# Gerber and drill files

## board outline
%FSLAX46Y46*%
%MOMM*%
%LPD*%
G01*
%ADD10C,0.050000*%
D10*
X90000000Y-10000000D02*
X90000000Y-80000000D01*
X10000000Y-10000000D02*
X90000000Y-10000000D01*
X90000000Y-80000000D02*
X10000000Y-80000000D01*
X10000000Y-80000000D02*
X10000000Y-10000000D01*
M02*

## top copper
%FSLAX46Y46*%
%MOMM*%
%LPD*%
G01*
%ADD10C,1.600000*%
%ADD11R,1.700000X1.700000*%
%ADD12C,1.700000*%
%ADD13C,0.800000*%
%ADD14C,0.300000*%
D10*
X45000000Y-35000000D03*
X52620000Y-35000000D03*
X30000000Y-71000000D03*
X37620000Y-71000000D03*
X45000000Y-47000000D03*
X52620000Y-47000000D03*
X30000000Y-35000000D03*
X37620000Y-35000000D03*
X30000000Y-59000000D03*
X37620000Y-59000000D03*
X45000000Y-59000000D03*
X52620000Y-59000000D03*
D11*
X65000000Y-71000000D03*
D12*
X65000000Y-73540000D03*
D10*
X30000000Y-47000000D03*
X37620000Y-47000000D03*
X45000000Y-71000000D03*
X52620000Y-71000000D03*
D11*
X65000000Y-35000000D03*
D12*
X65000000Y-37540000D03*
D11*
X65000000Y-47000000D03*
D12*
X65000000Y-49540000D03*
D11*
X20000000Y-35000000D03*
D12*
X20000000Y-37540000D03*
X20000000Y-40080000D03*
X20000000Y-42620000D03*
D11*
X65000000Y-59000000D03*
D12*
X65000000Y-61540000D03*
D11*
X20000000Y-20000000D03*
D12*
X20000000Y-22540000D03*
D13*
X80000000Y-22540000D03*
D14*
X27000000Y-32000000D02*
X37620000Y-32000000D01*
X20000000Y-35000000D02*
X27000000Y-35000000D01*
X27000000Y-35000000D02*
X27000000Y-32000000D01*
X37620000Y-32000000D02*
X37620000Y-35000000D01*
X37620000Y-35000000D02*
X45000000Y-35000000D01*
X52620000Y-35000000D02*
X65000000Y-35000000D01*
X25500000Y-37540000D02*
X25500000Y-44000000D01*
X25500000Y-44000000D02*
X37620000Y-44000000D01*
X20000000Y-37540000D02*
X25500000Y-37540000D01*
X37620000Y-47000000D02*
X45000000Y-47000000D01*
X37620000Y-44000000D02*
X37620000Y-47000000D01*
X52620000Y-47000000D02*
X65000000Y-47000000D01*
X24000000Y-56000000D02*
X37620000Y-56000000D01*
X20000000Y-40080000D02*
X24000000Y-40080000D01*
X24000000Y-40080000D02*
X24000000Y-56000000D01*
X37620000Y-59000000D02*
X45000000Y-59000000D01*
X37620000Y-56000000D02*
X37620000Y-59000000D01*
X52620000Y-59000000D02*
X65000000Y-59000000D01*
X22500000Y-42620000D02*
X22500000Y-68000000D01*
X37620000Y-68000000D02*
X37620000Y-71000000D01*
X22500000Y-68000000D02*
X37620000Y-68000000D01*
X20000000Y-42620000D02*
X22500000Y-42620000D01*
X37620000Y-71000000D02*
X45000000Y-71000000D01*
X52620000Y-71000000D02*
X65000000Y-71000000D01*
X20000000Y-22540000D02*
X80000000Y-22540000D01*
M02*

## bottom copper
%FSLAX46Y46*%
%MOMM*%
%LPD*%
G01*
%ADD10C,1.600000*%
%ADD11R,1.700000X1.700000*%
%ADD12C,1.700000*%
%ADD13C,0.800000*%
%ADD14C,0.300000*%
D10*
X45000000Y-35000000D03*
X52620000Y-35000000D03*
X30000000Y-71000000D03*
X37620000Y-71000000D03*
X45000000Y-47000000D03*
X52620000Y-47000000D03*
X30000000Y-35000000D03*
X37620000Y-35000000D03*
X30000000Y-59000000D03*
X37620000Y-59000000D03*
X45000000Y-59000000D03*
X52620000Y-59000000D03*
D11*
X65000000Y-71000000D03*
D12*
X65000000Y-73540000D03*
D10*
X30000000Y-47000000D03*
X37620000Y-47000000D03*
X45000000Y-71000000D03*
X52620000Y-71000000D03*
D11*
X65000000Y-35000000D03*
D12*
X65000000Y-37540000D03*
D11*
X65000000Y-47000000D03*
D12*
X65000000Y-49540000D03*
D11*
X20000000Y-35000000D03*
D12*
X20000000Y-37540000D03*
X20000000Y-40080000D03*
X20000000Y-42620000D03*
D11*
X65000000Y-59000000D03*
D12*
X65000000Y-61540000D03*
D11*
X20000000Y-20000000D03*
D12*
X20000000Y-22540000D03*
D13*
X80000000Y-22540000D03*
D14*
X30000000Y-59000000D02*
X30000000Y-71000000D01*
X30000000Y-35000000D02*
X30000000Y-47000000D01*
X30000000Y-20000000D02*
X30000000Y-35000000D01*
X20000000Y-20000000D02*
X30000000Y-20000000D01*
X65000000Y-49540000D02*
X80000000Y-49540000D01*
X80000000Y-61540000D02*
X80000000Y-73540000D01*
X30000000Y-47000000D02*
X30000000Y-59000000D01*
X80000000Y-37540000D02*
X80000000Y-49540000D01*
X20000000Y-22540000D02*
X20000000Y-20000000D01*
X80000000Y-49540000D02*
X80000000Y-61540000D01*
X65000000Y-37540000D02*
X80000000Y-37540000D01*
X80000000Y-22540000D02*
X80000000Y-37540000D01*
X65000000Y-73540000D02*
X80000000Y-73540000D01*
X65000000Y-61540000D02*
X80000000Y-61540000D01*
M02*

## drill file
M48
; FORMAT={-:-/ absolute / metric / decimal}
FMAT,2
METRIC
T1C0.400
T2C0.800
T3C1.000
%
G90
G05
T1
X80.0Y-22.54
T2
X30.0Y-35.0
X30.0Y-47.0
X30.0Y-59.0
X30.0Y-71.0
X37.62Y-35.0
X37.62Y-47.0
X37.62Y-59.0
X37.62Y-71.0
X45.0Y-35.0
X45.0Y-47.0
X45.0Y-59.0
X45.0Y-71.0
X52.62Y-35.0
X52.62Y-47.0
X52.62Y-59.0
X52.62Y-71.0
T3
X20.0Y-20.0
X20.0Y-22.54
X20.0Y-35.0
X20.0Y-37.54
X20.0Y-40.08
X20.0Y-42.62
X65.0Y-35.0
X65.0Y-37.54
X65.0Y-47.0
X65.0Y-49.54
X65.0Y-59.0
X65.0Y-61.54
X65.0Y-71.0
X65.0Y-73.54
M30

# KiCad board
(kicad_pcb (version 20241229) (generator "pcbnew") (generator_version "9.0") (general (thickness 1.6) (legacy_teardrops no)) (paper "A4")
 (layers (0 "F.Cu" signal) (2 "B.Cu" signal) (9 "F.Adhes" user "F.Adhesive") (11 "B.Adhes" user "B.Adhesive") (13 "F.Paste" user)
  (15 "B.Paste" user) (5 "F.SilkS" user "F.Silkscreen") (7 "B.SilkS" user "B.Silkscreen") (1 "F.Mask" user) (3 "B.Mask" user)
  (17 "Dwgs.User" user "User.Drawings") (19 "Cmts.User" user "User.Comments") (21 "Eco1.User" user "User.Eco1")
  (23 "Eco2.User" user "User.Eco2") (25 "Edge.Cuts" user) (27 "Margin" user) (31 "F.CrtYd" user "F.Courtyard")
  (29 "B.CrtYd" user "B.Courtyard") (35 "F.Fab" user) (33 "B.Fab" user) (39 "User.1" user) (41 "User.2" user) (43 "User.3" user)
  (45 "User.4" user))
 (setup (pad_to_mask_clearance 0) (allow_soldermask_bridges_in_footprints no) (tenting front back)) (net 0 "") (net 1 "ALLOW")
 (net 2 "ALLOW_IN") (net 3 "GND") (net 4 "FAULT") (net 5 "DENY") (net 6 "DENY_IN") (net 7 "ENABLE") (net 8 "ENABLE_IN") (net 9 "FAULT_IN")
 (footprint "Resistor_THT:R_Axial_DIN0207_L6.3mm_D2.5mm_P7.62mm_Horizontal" (layer "F.Cu") (at 45 35)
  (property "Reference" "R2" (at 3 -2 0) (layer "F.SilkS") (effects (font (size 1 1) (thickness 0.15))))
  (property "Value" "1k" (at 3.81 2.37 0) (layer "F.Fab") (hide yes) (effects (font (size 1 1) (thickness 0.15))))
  (pad "1" thru_hole circle (at 0 0) (size 1.6 1.6) (drill 0.8) (layers "*.Cu" "*.Mask") (remove_unused_layers no) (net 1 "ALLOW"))
  (pad "2" thru_hole circle (at 7.62 0) (size 1.6 1.6) (drill 0.8) (layers "*.Cu" "*.Mask") (remove_unused_layers no) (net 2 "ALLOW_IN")))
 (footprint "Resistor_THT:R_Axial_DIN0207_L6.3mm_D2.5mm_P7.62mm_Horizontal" (layer "F.Cu") (at 30 71)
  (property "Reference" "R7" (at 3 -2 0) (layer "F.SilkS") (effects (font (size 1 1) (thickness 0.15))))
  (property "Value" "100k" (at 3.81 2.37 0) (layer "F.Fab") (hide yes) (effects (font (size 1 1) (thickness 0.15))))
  (pad "1" thru_hole circle (at 0 0) (size 1.6 1.6) (drill 0.8) (layers "*.Cu" "*.Mask") (remove_unused_layers no) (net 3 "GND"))
  (pad "2" thru_hole circle (at 7.62 0) (size 1.6 1.6) (drill 0.8) (layers "*.Cu" "*.Mask") (remove_unused_layers no) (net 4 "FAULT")))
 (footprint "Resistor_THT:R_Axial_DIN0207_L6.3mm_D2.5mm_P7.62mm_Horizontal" (layer "F.Cu") (at 45 47)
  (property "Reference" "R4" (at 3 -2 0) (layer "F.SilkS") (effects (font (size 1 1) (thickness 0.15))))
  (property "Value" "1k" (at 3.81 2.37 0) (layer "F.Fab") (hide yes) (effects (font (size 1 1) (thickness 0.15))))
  (pad "1" thru_hole circle (at 0 0) (size 1.6 1.6) (drill 0.8) (layers "*.Cu" "*.Mask") (remove_unused_layers no) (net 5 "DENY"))
  (pad "2" thru_hole circle (at 7.62 0) (size 1.6 1.6) (drill 0.8) (layers "*.Cu" "*.Mask") (remove_unused_layers no) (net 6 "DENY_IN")))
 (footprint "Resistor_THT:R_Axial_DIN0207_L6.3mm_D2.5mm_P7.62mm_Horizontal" (layer "F.Cu") (at 30 35)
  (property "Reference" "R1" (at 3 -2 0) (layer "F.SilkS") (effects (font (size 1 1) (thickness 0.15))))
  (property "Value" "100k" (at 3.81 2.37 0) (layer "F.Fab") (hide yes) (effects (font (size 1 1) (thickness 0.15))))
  (pad "1" thru_hole circle (at 0 0) (size 1.6 1.6) (drill 0.8) (layers "*.Cu" "*.Mask") (remove_unused_layers no) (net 3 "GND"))
  (pad "2" thru_hole circle (at 7.62 0) (size 1.6 1.6) (drill 0.8) (layers "*.Cu" "*.Mask") (remove_unused_layers no) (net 1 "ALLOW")))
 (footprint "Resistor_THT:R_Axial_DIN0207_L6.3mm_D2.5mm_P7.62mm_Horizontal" (layer "F.Cu") (at 30 59)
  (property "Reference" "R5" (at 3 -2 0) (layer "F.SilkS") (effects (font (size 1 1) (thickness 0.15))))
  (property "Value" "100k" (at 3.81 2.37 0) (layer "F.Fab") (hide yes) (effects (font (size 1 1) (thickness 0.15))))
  (pad "1" thru_hole circle (at 0 0) (size 1.6 1.6) (drill 0.8) (layers "*.Cu" "*.Mask") (remove_unused_layers no) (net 3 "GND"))
  (pad "2" thru_hole circle (at 7.62 0) (size 1.6 1.6) (drill 0.8) (layers "*.Cu" "*.Mask") (remove_unused_layers no) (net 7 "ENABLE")))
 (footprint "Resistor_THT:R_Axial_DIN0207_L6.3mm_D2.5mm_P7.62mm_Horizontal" (layer "F.Cu") (at 45 59)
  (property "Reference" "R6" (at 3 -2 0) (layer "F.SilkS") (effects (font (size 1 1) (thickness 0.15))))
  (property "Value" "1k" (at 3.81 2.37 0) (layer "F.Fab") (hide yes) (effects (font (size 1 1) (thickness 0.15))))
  (pad "1" thru_hole circle (at 0 0) (size 1.6 1.6) (drill 0.8) (layers "*.Cu" "*.Mask") (remove_unused_layers no) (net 7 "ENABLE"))
  (pad "2" thru_hole circle (at 7.62 0) (size 1.6 1.6) (drill 0.8) (layers "*.Cu" "*.Mask") (remove_unused_layers no) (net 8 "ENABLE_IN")))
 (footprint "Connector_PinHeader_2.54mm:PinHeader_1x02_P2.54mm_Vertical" (layer "F.Cu") (at 65 71)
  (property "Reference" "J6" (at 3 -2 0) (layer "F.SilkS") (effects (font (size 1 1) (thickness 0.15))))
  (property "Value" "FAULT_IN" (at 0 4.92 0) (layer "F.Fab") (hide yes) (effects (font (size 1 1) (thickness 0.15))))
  (pad "1" thru_hole rect (at 0 0) (size 1.7 1.7) (drill 1) (layers "*.Cu" "*.Mask") (remove_unused_layers no) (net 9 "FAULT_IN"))
  (pad "2" thru_hole circle (at 0 2.54) (size 1.7 1.7) (drill 1) (layers "*.Cu" "*.Mask") (remove_unused_layers no) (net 3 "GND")))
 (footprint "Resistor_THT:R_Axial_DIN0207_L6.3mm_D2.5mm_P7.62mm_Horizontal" (layer "F.Cu") (at 30 47)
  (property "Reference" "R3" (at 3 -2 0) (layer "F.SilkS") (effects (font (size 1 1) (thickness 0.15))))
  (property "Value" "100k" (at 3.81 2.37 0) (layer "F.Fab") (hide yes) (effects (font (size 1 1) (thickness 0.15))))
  (pad "1" thru_hole circle (at 0 0) (size 1.6 1.6) (drill 0.8) (layers "*.Cu" "*.Mask") (remove_unused_layers no) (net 3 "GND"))
  (pad "2" thru_hole circle (at 7.62 0) (size 1.6 1.6) (drill 0.8) (layers "*.Cu" "*.Mask") (remove_unused_layers no) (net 5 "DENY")))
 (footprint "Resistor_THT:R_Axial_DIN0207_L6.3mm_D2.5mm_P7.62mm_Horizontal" (layer "F.Cu") (at 45 71)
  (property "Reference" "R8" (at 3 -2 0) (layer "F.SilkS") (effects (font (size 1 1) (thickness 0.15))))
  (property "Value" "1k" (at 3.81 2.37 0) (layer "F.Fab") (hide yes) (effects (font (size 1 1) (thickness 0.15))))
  (pad "1" thru_hole circle (at 0 0) (size 1.6 1.6) (drill 0.8) (layers "*.Cu" "*.Mask") (remove_unused_layers no) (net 4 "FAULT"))
  (pad "2" thru_hole circle (at 7.62 0) (size 1.6 1.6) (drill 0.8) (layers "*.Cu" "*.Mask") (remove_unused_layers no) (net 9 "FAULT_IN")))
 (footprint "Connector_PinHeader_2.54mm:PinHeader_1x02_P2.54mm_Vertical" (layer "F.Cu") (at 65 35)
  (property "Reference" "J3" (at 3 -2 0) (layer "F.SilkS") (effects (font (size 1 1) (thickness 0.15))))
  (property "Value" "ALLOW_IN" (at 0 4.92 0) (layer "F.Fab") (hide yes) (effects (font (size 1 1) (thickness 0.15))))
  (pad "1" thru_hole rect (at 0 0) (size 1.7 1.7) (drill 1) (layers "*.Cu" "*.Mask") (remove_unused_layers no) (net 2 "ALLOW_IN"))
  (pad "2" thru_hole circle (at 0 2.54) (size 1.7 1.7) (drill 1) (layers "*.Cu" "*.Mask") (remove_unused_layers no) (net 3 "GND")))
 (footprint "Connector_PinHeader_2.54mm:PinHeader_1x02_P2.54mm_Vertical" (layer "F.Cu") (at 65 47)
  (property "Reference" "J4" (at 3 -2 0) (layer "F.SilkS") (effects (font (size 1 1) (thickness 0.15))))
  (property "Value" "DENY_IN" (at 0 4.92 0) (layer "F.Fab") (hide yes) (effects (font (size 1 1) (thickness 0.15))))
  (pad "1" thru_hole rect (at 0 0) (size 1.7 1.7) (drill 1) (layers "*.Cu" "*.Mask") (remove_unused_layers no) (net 6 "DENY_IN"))
  (pad "2" thru_hole circle (at 0 2.54) (size 1.7 1.7) (drill 1) (layers "*.Cu" "*.Mask") (remove_unused_layers no) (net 3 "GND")))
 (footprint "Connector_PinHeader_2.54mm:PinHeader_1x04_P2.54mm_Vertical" (layer "F.Cu") (at 20 35)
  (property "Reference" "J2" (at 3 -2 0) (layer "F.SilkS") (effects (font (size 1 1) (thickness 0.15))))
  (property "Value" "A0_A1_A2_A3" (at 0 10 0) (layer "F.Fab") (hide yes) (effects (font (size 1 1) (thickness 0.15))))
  (pad "1" thru_hole rect (at 0 0) (size 1.7 1.7) (drill 1) (layers "*.Cu" "*.Mask") (remove_unused_layers no) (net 1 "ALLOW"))
  (pad "2" thru_hole circle (at 0 2.54) (size 1.7 1.7) (drill 1) (layers "*.Cu" "*.Mask") (remove_unused_layers no) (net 5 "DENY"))
  (pad "3" thru_hole circle (at 0 5.08) (size 1.7 1.7) (drill 1) (layers "*.Cu" "*.Mask") (remove_unused_layers no) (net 7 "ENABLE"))
  (pad "4" thru_hole circle (at 0 7.62) (size 1.7 1.7) (drill 1) (layers "*.Cu" "*.Mask") (remove_unused_layers no) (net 4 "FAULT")))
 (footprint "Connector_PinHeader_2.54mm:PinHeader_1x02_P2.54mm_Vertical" (layer "F.Cu") (at 65 59)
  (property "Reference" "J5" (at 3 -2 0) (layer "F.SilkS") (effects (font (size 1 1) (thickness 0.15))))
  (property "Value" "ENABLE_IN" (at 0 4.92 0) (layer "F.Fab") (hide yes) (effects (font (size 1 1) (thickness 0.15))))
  (pad "1" thru_hole rect (at 0 0) (size 1.7 1.7) (drill 1) (layers "*.Cu" "*.Mask") (remove_unused_layers no) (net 8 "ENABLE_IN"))
  (pad "2" thru_hole circle (at 0 2.54) (size 1.7 1.7) (drill 1) (layers "*.Cu" "*.Mask") (remove_unused_layers no) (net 3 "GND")))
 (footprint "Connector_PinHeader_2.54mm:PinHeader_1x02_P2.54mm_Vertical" (layer "F.Cu") (at 20 20)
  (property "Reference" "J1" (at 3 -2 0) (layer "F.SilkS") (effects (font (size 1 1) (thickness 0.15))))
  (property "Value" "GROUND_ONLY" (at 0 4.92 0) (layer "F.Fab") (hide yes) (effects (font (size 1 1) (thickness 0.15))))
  (pad "1" thru_hole rect (at 0 0) (size 1.7 1.7) (drill 1) (layers "*.Cu" "*.Mask") (remove_unused_layers no) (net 3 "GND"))
  (pad "2" thru_hole circle (at 0 2.54) (size 1.7 1.7) (drill 1) (layers "*.Cu" "*.Mask") (remove_unused_layers no) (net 3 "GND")))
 (gr_line (start 90 10) (end 90 80) (stroke (width 0.05) (type default)) (layer "Edge.Cuts"))
 (gr_line (start 10 10) (end 90 10) (stroke (width 0.05) (type default)) (layer "Edge.Cuts"))
 (gr_line (start 90 80) (end 10 80) (stroke (width 0.05) (type default)) (layer "Edge.Cuts"))
 (gr_line (start 10 80) (end 10 10) (stroke (width 0.05) (type default)) (layer "Edge.Cuts"))
 (segment (start 27 32) (end 37.62 32) (width 0.3) (layer "F.Cu") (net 1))
 (segment (start 20 35) (end 27 35) (width 0.3) (layer "F.Cu") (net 1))
 (segment (start 27 35) (end 27 32) (width 0.3) (layer "F.Cu") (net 1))
 (segment (start 37.62 32) (end 37.62 35) (width 0.3) (layer "F.Cu") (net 1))
 (segment (start 37.62 35) (end 45 35) (width 0.3) (layer "F.Cu") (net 1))
 (segment (start 52.62 35) (end 65 35) (width 0.3) (layer "F.Cu") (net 2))
 (segment (start 25.5 37.54) (end 25.5 44) (width 0.3) (layer "F.Cu") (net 5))
 (segment (start 25.5 44) (end 37.62 44) (width 0.3) (layer "F.Cu") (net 5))
 (segment (start 20 37.54) (end 25.5 37.54) (width 0.3) (layer "F.Cu") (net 5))
 (segment (start 37.62 47) (end 45 47) (width 0.3) (layer "F.Cu") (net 5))
 (segment (start 37.62 44) (end 37.62 47) (width 0.3) (layer "F.Cu") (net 5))
 (segment (start 52.62 47) (end 65 47) (width 0.3) (layer "F.Cu") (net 6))
 (segment (start 24 56) (end 37.62 56) (width 0.3) (layer "F.Cu") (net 7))
 (segment (start 20 40.08) (end 24 40.08) (width 0.3) (layer "F.Cu") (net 7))
 (segment (start 24 40.08) (end 24 56) (width 0.3) (layer "F.Cu") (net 7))
 (segment (start 37.62 59) (end 45 59) (width 0.3) (layer "F.Cu") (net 7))
 (segment (start 37.62 56) (end 37.62 59) (width 0.3) (layer "F.Cu") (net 7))
 (segment (start 52.62 59) (end 65 59) (width 0.3) (layer "F.Cu") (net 8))
 (segment (start 22.5 42.62) (end 22.5 68) (width 0.3) (layer "F.Cu") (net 4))
 (segment (start 37.62 68) (end 37.62 71) (width 0.3) (layer "F.Cu") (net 4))
 (segment (start 22.5 68) (end 37.62 68) (width 0.3) (layer "F.Cu") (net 4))
 (segment (start 20 42.62) (end 22.5 42.62) (width 0.3) (layer "F.Cu") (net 4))
 (segment (start 37.62 71) (end 45 71) (width 0.3) (layer "F.Cu") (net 4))
 (segment (start 52.62 71) (end 65 71) (width 0.3) (layer "F.Cu") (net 9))
 (segment (start 20 22.54) (end 80 22.54) (width 0.3) (layer "F.Cu") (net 3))
 (via (at 80 22.54) (size 0.8) (drill 0.4) (layers "F.Cu" "B.Cu") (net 3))
 (segment (start 30 59) (end 30 71) (width 0.3) (layer "B.Cu") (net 3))
 (segment (start 30 35) (end 30 47) (width 0.3) (layer "B.Cu") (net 3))
 (segment (start 30 20) (end 30 35) (width 0.3) (layer "B.Cu") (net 3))
 (segment (start 20 20) (end 30 20) (width 0.3) (layer "B.Cu") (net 3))
 (segment (start 65 49.54) (end 80 49.54) (width 0.3) (layer "B.Cu") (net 3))
 (segment (start 80 61.54) (end 80 73.54) (width 0.3) (layer "B.Cu") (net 3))
 (segment (start 30 47) (end 30 59) (width 0.3) (layer "B.Cu") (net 3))
 (segment (start 80 37.54) (end 80 49.54) (width 0.3) (layer "B.Cu") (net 3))
 (segment (start 20 22.54) (end 20 20) (width 0.3) (layer "B.Cu") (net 3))
 (segment (start 80 49.54) (end 80 61.54) (width 0.3) (layer "B.Cu") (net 3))
 (segment (start 65 37.54) (end 80 37.54) (width 0.3) (layer "B.Cu") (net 3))
 (segment (start 80 22.54) (end 80 37.54) (width 0.3) (layer "B.Cu") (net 3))
 (segment (start 65 73.54) (end 80 73.54) (width 0.3) (layer "B.Cu") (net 3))
 (segment (start 65 61.54) (end 80 61.54) (width 0.3) (layer "B.Cu") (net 3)))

